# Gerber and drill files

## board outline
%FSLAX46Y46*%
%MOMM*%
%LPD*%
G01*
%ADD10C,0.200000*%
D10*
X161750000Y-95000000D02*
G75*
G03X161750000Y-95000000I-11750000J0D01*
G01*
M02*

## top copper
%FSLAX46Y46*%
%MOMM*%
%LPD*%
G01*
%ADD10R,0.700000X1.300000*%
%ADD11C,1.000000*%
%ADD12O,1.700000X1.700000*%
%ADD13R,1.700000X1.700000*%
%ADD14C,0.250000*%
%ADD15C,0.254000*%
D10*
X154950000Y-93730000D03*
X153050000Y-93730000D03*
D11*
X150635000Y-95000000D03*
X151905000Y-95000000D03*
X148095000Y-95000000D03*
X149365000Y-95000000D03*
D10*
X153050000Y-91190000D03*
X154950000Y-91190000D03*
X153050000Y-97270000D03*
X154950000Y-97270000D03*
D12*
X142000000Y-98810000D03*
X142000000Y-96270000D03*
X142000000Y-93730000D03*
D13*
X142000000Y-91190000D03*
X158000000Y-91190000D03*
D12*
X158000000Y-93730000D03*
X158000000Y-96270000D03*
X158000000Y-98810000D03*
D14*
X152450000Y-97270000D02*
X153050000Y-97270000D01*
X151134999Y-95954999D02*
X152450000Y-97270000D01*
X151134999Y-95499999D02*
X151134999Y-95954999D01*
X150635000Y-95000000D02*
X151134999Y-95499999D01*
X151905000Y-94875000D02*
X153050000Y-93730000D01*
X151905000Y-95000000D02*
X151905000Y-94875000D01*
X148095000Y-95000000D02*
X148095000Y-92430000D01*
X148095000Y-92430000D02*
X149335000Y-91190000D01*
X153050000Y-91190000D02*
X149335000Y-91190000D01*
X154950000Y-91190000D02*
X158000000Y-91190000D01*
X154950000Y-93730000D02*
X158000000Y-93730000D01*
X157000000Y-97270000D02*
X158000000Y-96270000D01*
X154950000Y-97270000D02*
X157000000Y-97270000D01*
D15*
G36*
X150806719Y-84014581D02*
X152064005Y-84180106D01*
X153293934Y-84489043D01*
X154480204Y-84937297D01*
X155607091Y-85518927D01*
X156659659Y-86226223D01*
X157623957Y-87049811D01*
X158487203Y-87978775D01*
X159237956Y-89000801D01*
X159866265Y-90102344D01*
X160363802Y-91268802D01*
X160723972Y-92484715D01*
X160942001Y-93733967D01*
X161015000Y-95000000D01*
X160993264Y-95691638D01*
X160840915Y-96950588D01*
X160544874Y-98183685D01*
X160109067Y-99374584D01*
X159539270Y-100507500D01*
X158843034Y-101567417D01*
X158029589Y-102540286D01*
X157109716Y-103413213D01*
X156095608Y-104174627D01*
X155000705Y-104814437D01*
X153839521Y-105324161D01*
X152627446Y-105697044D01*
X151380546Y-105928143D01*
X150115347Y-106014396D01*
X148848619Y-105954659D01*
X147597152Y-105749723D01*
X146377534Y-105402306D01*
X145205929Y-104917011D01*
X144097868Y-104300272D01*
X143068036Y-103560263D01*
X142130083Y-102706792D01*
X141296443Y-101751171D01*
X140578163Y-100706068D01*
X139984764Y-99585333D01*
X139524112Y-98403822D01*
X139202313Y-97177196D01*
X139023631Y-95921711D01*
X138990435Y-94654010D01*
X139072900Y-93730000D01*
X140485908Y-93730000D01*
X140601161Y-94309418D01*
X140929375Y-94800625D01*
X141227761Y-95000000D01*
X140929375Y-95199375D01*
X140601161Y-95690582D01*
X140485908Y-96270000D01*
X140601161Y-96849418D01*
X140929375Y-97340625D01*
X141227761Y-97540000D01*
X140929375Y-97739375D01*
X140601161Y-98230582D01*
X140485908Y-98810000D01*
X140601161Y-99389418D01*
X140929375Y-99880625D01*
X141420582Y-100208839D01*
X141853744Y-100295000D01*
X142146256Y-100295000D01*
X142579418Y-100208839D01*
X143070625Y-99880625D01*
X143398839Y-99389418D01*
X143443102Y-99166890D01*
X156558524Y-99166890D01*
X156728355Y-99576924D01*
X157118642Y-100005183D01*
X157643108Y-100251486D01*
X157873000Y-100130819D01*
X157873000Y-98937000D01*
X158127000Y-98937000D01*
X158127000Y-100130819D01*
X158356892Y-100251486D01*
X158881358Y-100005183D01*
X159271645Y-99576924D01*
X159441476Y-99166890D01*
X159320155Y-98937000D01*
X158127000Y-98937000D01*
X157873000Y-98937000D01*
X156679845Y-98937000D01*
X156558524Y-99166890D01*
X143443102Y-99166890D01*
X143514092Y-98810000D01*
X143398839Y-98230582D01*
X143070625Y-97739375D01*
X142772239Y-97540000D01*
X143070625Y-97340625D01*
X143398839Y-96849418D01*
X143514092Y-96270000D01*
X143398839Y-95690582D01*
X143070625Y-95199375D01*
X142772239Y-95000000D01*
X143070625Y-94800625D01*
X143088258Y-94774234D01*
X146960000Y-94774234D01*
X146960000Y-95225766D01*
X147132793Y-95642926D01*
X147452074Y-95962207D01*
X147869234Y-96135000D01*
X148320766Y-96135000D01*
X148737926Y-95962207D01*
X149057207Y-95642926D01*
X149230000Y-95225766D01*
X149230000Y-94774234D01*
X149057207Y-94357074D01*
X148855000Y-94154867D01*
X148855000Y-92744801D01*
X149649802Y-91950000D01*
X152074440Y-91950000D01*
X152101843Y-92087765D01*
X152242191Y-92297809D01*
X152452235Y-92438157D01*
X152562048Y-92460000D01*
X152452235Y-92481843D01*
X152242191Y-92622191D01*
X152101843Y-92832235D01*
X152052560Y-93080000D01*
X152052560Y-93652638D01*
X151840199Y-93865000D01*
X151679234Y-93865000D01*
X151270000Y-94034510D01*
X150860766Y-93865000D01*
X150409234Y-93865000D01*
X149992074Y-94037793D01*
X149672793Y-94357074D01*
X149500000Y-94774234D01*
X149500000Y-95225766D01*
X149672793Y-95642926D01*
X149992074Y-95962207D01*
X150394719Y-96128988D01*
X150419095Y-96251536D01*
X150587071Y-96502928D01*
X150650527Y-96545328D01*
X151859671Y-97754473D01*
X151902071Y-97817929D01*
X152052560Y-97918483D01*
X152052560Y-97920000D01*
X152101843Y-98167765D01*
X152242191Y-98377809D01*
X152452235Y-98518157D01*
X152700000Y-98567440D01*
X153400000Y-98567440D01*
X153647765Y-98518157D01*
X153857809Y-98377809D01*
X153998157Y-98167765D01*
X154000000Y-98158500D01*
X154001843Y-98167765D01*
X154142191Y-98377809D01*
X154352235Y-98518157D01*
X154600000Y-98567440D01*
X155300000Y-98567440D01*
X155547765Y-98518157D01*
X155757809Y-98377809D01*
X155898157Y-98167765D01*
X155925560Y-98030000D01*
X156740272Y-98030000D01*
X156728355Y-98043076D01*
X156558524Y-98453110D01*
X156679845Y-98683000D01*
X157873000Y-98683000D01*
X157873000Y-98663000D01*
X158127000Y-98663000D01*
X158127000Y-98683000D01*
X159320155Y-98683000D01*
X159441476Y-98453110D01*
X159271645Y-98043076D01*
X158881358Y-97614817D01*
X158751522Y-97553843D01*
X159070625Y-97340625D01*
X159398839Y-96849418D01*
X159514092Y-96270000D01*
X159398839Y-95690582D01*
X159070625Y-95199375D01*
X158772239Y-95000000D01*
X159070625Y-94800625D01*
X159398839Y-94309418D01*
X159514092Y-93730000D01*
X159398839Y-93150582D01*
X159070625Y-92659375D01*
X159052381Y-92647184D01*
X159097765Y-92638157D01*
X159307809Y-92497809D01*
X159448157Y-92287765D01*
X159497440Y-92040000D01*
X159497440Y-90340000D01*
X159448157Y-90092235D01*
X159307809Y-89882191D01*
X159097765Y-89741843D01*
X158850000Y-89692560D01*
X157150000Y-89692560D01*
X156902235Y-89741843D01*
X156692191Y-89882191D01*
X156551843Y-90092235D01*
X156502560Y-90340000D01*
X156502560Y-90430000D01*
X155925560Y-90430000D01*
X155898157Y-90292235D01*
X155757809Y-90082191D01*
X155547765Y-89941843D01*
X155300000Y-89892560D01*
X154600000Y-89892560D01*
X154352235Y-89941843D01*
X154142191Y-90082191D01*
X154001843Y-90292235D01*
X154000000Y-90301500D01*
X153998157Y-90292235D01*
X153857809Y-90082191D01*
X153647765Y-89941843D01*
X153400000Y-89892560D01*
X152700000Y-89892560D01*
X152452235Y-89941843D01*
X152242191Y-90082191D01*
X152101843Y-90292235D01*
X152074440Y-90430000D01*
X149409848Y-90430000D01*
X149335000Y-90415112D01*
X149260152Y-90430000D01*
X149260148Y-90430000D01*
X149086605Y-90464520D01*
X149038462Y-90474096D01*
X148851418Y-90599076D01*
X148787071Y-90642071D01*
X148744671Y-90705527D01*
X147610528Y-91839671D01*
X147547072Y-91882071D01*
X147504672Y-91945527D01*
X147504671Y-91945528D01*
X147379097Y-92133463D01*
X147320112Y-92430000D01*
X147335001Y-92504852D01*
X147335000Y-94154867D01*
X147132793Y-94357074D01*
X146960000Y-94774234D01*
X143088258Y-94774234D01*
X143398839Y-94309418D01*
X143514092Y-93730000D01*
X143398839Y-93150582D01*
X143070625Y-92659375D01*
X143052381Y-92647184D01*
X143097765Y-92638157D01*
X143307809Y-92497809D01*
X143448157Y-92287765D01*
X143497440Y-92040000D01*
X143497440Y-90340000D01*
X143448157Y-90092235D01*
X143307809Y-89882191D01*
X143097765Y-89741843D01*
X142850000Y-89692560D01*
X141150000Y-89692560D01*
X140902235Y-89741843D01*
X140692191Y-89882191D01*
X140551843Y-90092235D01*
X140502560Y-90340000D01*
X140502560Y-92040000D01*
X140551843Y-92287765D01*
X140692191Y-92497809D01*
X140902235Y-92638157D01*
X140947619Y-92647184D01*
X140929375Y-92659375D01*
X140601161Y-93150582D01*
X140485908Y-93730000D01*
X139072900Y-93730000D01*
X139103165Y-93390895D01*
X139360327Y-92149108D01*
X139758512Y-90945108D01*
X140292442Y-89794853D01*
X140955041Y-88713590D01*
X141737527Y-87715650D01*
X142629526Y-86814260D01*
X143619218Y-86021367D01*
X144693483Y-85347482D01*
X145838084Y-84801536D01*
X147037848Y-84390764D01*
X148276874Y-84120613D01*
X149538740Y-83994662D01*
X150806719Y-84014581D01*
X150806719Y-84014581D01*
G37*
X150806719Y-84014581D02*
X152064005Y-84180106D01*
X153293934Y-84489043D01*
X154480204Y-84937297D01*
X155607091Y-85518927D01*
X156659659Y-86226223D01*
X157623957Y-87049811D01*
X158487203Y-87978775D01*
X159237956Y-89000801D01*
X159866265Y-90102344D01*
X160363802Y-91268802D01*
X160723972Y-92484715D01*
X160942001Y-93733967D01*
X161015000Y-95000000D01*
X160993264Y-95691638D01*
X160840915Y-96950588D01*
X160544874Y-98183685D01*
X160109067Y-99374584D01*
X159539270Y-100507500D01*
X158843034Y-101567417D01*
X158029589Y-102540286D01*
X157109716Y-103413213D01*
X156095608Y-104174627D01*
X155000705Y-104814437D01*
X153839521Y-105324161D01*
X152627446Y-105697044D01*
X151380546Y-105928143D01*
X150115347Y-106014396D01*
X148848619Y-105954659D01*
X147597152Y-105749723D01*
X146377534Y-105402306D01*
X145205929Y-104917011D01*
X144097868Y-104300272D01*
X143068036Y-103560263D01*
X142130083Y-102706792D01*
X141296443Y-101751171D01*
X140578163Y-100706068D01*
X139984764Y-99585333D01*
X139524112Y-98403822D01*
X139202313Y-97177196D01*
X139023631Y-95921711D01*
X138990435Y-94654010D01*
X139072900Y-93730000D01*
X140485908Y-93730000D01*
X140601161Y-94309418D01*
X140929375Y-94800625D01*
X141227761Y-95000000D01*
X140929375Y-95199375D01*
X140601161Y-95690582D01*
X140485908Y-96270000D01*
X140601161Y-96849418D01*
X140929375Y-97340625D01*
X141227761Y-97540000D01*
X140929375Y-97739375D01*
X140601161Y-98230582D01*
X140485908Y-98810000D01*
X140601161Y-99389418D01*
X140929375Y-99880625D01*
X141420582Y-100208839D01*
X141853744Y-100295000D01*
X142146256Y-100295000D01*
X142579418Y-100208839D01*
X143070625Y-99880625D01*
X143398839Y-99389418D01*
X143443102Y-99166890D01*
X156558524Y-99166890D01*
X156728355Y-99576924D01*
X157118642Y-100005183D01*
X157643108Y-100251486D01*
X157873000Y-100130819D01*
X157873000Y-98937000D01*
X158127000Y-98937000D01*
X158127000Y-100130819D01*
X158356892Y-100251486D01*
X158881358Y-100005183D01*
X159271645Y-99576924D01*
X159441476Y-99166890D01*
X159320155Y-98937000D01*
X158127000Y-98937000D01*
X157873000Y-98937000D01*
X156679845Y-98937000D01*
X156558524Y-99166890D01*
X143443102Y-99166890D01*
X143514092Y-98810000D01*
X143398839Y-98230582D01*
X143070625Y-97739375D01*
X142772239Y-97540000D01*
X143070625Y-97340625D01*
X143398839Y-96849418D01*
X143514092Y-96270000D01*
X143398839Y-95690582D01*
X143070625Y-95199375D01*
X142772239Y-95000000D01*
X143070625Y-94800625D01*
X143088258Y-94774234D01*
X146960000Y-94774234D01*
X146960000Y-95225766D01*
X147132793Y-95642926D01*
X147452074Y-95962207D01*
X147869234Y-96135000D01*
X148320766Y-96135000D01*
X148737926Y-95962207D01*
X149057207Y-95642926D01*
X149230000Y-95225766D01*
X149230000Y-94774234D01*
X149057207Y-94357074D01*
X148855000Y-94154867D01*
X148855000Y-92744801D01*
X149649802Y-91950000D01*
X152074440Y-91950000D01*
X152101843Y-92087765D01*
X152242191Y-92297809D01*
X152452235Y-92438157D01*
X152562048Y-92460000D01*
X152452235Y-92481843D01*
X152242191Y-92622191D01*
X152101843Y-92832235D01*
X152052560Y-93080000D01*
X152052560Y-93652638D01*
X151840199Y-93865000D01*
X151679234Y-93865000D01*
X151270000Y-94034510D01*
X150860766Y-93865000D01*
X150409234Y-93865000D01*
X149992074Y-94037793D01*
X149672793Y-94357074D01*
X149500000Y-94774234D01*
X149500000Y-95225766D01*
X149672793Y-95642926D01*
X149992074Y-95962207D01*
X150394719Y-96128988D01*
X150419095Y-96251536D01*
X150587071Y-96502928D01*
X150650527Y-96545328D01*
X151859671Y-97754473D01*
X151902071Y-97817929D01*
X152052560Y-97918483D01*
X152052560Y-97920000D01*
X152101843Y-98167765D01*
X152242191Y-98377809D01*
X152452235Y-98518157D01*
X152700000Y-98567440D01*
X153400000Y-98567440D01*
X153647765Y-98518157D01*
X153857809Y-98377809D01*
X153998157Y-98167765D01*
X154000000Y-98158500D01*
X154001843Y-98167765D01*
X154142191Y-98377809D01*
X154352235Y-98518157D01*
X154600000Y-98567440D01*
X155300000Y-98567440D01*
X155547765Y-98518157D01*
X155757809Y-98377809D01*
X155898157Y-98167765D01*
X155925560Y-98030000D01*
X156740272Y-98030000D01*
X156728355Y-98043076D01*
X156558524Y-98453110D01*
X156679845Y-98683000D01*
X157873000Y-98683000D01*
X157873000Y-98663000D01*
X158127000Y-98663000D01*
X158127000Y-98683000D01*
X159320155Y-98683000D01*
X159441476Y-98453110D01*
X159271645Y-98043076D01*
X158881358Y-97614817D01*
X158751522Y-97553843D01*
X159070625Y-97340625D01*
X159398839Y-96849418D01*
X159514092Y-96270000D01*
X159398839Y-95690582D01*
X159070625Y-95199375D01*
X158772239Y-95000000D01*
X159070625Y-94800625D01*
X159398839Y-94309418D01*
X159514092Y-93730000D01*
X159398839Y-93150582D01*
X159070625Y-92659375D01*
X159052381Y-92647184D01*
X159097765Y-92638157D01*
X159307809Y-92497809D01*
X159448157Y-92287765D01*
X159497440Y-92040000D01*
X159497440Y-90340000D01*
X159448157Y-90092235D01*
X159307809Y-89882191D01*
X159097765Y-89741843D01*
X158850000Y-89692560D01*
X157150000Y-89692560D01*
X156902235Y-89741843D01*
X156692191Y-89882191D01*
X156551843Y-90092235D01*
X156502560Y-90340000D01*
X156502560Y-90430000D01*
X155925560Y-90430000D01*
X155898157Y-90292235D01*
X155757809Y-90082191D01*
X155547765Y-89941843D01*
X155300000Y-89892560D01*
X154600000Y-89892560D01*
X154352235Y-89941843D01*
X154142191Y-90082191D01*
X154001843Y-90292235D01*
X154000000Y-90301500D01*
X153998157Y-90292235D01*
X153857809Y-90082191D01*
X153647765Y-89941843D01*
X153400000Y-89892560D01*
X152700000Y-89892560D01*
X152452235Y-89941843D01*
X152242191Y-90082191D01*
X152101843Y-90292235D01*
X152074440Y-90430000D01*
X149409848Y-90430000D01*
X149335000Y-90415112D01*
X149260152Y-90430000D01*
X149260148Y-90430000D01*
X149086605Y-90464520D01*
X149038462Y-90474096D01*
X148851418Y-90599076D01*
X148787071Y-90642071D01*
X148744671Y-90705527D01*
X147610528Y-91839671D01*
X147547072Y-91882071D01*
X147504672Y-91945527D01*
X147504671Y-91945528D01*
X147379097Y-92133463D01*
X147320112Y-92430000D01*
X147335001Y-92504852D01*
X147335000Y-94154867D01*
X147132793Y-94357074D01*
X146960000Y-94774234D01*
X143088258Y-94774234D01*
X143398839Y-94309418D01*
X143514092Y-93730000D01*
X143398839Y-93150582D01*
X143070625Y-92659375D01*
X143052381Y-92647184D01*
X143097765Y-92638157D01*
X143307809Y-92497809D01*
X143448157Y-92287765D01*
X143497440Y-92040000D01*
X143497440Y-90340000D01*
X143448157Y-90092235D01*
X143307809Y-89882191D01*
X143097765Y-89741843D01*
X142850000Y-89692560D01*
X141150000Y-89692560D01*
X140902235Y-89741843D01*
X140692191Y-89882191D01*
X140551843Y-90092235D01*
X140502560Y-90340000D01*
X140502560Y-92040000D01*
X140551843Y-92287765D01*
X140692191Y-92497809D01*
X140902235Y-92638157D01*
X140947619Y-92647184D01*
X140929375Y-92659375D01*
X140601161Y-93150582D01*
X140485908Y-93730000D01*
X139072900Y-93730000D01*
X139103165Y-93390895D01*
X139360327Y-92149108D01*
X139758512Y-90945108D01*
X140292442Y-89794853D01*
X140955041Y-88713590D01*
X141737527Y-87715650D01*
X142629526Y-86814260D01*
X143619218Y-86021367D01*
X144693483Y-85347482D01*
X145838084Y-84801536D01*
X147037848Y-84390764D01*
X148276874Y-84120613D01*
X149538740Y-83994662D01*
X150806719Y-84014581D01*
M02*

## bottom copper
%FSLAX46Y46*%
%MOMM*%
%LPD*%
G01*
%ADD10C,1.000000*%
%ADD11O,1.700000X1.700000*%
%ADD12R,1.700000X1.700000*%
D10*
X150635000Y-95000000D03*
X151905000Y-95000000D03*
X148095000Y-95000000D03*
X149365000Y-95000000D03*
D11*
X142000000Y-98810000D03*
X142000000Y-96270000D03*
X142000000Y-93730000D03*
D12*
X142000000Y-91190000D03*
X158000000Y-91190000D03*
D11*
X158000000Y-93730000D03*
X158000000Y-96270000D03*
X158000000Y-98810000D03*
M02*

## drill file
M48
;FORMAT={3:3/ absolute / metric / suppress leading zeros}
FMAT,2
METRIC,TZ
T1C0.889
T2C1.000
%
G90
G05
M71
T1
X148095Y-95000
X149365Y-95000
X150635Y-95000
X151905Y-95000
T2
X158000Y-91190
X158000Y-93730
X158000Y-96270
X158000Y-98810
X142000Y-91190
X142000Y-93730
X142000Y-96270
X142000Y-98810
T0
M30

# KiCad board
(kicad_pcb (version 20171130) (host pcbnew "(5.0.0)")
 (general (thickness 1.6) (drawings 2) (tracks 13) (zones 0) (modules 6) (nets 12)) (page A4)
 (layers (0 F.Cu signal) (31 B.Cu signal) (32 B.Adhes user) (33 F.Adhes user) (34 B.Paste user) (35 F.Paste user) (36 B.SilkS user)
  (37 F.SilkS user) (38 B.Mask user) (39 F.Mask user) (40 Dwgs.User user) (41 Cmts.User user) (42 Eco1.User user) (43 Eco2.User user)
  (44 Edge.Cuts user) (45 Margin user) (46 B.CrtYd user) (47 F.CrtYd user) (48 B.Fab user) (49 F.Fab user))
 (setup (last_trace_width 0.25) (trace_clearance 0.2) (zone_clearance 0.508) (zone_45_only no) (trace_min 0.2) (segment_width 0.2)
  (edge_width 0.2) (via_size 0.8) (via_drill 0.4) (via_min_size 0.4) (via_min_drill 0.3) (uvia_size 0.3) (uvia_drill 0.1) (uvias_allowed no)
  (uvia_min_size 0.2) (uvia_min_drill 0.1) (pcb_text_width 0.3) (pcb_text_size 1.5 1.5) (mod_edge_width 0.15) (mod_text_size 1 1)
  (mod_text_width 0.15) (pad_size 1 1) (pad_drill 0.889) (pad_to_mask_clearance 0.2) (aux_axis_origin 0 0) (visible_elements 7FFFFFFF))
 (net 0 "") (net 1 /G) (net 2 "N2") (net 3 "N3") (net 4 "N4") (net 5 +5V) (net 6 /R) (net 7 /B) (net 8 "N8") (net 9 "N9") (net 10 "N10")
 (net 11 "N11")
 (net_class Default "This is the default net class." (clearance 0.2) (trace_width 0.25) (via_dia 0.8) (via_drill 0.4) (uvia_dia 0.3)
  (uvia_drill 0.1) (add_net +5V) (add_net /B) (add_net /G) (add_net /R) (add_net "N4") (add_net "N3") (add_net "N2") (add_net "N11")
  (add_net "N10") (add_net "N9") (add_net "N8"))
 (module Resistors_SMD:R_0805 (layer F.Cu) (at 154 93.73)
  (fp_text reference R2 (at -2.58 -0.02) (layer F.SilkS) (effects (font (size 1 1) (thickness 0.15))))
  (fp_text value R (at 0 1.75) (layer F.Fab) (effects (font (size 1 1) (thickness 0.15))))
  (pad 2 smd rect (at 0.95 0) (size 0.7 1.3) (layers F.Cu F.Paste F.Mask) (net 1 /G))
  (pad 1 smd rect (at -0.95 0) (size 0.7 1.3) (layers F.Cu F.Paste F.Mask) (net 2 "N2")))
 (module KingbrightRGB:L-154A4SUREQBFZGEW (layer F.Cu) (at 150 95)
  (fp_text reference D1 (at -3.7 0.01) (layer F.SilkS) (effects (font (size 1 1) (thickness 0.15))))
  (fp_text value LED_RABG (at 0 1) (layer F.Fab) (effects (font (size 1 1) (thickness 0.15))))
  (pad 3 thru_hole circle (at 0.635 0) (size 1 1) (drill 0.889) (layers *.Cu *.Mask) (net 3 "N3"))
  (pad 4 thru_hole circle (at 1.905 0) (size 1 1) (drill 0.889) (layers *.Cu *.Mask) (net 2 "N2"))
  (pad 1 thru_hole circle (at -1.905 0) (size 1 1) (drill 0.889) (layers *.Cu *.Mask) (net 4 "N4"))
  (pad 2 thru_hole circle (at -0.635 0) (size 1 1) (drill 0.889) (layers *.Cu *.Mask) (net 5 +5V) (zone_connect 2)))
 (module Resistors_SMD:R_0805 (layer F.Cu) (at 154 91.19)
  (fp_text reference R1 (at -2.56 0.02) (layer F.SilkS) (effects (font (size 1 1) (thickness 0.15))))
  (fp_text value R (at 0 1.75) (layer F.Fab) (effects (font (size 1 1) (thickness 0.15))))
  (pad 1 smd rect (at -0.95 0) (size 0.7 1.3) (layers F.Cu F.Paste F.Mask) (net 4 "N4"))
  (pad 2 smd rect (at 0.95 0) (size 0.7 1.3) (layers F.Cu F.Paste F.Mask) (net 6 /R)))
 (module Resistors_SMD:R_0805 (layer F.Cu) (at 154 97.27)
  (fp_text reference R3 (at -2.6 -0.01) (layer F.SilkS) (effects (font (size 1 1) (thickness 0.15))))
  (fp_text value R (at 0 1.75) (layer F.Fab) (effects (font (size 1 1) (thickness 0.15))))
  (pad 1 smd rect (at -0.95 0) (size 0.7 1.3) (layers F.Cu F.Paste F.Mask) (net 3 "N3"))
  (pad 2 smd rect (at 0.95 0) (size 0.7 1.3) (layers F.Cu F.Paste F.Mask) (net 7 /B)))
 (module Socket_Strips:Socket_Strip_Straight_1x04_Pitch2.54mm (layer F.Cu) (at 142 91.19)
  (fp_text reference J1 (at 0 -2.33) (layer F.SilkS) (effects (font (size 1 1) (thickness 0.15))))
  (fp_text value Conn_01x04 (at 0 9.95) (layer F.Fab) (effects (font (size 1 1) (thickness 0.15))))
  (pad 4 thru_hole oval (at 0 7.62) (size 1.7 1.7) (drill 1) (layers *.Cu *.Mask) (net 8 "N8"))
  (pad 3 thru_hole oval (at 0 5.08) (size 1.7 1.7) (drill 1) (layers *.Cu *.Mask) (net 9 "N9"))
  (pad 2 thru_hole oval (at 0 2.54) (size 1.7 1.7) (drill 1) (layers *.Cu *.Mask) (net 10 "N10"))
  (pad 1 thru_hole rect (at 0 0) (size 1.7 1.7) (drill 1) (layers *.Cu *.Mask) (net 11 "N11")))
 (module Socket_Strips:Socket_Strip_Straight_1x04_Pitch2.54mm (layer F.Cu) (at 158 91.19)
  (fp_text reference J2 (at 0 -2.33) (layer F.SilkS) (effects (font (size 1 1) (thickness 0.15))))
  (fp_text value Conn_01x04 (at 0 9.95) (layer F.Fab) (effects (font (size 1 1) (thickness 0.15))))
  (pad 1 thru_hole rect (at 0 0) (size 1.7 1.7) (drill 1) (layers *.Cu *.Mask) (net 6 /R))
  (pad 2 thru_hole oval (at 0 2.54) (size 1.7 1.7) (drill 1) (layers *.Cu *.Mask) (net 1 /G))
  (pad 3 thru_hole oval (at 0 5.08) (size 1.7 1.7) (drill 1) (layers *.Cu *.Mask) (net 7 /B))
  (pad 4 thru_hole oval (at 0 7.62) (size 1.7 1.7) (drill 1) (layers *.Cu *.Mask) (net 5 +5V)))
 (gr_circle (center 150 95) (end 161.75 95) (layer Edge.Cuts) (width 0.2))
 (segment (start 152.45 97.27) (end 153.05 97.27) (width 0.25) (layer F.Cu) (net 3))
 (segment (start 151.134999 95.954999) (end 152.45 97.27) (width 0.25) (layer F.Cu) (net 3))
 (segment (start 151.134999 95.499999) (end 151.134999 95.954999) (width 0.25) (layer F.Cu) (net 3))
 (segment (start 150.635 95) (end 151.134999 95.499999) (width 0.25) (layer F.Cu) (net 3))
 (segment (start 151.905 94.875) (end 153.05 93.73) (width 0.25) (layer F.Cu) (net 2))
 (segment (start 151.905 95) (end 151.905 94.875) (width 0.25) (layer F.Cu) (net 2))
 (segment (start 148.095 95) (end 148.095 92.43) (width 0.25) (layer F.Cu) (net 4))
 (segment (start 148.095 92.43) (end 149.335 91.19) (width 0.25) (layer F.Cu) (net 4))
 (segment (start 153.05 91.19) (end 149.335 91.19) (width 0.25) (layer F.Cu) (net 4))
 (segment (start 154.95 91.19) (end 158 91.19) (width 0.25) (layer F.Cu) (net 6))
 (segment (start 154.95 93.73) (end 158 93.73) (width 0.25) (layer F.Cu) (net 1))
 (segment (start 157 97.27) (end 158 96.27) (width 0.25) (layer F.Cu) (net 7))
 (segment (start 154.95 97.27) (end 157 97.27) (width 0.25) (layer F.Cu) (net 7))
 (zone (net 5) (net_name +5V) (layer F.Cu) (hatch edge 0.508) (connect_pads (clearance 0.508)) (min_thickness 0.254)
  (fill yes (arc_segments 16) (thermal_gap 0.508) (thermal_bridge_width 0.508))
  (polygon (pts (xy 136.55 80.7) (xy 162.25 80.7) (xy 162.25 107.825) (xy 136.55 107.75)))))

